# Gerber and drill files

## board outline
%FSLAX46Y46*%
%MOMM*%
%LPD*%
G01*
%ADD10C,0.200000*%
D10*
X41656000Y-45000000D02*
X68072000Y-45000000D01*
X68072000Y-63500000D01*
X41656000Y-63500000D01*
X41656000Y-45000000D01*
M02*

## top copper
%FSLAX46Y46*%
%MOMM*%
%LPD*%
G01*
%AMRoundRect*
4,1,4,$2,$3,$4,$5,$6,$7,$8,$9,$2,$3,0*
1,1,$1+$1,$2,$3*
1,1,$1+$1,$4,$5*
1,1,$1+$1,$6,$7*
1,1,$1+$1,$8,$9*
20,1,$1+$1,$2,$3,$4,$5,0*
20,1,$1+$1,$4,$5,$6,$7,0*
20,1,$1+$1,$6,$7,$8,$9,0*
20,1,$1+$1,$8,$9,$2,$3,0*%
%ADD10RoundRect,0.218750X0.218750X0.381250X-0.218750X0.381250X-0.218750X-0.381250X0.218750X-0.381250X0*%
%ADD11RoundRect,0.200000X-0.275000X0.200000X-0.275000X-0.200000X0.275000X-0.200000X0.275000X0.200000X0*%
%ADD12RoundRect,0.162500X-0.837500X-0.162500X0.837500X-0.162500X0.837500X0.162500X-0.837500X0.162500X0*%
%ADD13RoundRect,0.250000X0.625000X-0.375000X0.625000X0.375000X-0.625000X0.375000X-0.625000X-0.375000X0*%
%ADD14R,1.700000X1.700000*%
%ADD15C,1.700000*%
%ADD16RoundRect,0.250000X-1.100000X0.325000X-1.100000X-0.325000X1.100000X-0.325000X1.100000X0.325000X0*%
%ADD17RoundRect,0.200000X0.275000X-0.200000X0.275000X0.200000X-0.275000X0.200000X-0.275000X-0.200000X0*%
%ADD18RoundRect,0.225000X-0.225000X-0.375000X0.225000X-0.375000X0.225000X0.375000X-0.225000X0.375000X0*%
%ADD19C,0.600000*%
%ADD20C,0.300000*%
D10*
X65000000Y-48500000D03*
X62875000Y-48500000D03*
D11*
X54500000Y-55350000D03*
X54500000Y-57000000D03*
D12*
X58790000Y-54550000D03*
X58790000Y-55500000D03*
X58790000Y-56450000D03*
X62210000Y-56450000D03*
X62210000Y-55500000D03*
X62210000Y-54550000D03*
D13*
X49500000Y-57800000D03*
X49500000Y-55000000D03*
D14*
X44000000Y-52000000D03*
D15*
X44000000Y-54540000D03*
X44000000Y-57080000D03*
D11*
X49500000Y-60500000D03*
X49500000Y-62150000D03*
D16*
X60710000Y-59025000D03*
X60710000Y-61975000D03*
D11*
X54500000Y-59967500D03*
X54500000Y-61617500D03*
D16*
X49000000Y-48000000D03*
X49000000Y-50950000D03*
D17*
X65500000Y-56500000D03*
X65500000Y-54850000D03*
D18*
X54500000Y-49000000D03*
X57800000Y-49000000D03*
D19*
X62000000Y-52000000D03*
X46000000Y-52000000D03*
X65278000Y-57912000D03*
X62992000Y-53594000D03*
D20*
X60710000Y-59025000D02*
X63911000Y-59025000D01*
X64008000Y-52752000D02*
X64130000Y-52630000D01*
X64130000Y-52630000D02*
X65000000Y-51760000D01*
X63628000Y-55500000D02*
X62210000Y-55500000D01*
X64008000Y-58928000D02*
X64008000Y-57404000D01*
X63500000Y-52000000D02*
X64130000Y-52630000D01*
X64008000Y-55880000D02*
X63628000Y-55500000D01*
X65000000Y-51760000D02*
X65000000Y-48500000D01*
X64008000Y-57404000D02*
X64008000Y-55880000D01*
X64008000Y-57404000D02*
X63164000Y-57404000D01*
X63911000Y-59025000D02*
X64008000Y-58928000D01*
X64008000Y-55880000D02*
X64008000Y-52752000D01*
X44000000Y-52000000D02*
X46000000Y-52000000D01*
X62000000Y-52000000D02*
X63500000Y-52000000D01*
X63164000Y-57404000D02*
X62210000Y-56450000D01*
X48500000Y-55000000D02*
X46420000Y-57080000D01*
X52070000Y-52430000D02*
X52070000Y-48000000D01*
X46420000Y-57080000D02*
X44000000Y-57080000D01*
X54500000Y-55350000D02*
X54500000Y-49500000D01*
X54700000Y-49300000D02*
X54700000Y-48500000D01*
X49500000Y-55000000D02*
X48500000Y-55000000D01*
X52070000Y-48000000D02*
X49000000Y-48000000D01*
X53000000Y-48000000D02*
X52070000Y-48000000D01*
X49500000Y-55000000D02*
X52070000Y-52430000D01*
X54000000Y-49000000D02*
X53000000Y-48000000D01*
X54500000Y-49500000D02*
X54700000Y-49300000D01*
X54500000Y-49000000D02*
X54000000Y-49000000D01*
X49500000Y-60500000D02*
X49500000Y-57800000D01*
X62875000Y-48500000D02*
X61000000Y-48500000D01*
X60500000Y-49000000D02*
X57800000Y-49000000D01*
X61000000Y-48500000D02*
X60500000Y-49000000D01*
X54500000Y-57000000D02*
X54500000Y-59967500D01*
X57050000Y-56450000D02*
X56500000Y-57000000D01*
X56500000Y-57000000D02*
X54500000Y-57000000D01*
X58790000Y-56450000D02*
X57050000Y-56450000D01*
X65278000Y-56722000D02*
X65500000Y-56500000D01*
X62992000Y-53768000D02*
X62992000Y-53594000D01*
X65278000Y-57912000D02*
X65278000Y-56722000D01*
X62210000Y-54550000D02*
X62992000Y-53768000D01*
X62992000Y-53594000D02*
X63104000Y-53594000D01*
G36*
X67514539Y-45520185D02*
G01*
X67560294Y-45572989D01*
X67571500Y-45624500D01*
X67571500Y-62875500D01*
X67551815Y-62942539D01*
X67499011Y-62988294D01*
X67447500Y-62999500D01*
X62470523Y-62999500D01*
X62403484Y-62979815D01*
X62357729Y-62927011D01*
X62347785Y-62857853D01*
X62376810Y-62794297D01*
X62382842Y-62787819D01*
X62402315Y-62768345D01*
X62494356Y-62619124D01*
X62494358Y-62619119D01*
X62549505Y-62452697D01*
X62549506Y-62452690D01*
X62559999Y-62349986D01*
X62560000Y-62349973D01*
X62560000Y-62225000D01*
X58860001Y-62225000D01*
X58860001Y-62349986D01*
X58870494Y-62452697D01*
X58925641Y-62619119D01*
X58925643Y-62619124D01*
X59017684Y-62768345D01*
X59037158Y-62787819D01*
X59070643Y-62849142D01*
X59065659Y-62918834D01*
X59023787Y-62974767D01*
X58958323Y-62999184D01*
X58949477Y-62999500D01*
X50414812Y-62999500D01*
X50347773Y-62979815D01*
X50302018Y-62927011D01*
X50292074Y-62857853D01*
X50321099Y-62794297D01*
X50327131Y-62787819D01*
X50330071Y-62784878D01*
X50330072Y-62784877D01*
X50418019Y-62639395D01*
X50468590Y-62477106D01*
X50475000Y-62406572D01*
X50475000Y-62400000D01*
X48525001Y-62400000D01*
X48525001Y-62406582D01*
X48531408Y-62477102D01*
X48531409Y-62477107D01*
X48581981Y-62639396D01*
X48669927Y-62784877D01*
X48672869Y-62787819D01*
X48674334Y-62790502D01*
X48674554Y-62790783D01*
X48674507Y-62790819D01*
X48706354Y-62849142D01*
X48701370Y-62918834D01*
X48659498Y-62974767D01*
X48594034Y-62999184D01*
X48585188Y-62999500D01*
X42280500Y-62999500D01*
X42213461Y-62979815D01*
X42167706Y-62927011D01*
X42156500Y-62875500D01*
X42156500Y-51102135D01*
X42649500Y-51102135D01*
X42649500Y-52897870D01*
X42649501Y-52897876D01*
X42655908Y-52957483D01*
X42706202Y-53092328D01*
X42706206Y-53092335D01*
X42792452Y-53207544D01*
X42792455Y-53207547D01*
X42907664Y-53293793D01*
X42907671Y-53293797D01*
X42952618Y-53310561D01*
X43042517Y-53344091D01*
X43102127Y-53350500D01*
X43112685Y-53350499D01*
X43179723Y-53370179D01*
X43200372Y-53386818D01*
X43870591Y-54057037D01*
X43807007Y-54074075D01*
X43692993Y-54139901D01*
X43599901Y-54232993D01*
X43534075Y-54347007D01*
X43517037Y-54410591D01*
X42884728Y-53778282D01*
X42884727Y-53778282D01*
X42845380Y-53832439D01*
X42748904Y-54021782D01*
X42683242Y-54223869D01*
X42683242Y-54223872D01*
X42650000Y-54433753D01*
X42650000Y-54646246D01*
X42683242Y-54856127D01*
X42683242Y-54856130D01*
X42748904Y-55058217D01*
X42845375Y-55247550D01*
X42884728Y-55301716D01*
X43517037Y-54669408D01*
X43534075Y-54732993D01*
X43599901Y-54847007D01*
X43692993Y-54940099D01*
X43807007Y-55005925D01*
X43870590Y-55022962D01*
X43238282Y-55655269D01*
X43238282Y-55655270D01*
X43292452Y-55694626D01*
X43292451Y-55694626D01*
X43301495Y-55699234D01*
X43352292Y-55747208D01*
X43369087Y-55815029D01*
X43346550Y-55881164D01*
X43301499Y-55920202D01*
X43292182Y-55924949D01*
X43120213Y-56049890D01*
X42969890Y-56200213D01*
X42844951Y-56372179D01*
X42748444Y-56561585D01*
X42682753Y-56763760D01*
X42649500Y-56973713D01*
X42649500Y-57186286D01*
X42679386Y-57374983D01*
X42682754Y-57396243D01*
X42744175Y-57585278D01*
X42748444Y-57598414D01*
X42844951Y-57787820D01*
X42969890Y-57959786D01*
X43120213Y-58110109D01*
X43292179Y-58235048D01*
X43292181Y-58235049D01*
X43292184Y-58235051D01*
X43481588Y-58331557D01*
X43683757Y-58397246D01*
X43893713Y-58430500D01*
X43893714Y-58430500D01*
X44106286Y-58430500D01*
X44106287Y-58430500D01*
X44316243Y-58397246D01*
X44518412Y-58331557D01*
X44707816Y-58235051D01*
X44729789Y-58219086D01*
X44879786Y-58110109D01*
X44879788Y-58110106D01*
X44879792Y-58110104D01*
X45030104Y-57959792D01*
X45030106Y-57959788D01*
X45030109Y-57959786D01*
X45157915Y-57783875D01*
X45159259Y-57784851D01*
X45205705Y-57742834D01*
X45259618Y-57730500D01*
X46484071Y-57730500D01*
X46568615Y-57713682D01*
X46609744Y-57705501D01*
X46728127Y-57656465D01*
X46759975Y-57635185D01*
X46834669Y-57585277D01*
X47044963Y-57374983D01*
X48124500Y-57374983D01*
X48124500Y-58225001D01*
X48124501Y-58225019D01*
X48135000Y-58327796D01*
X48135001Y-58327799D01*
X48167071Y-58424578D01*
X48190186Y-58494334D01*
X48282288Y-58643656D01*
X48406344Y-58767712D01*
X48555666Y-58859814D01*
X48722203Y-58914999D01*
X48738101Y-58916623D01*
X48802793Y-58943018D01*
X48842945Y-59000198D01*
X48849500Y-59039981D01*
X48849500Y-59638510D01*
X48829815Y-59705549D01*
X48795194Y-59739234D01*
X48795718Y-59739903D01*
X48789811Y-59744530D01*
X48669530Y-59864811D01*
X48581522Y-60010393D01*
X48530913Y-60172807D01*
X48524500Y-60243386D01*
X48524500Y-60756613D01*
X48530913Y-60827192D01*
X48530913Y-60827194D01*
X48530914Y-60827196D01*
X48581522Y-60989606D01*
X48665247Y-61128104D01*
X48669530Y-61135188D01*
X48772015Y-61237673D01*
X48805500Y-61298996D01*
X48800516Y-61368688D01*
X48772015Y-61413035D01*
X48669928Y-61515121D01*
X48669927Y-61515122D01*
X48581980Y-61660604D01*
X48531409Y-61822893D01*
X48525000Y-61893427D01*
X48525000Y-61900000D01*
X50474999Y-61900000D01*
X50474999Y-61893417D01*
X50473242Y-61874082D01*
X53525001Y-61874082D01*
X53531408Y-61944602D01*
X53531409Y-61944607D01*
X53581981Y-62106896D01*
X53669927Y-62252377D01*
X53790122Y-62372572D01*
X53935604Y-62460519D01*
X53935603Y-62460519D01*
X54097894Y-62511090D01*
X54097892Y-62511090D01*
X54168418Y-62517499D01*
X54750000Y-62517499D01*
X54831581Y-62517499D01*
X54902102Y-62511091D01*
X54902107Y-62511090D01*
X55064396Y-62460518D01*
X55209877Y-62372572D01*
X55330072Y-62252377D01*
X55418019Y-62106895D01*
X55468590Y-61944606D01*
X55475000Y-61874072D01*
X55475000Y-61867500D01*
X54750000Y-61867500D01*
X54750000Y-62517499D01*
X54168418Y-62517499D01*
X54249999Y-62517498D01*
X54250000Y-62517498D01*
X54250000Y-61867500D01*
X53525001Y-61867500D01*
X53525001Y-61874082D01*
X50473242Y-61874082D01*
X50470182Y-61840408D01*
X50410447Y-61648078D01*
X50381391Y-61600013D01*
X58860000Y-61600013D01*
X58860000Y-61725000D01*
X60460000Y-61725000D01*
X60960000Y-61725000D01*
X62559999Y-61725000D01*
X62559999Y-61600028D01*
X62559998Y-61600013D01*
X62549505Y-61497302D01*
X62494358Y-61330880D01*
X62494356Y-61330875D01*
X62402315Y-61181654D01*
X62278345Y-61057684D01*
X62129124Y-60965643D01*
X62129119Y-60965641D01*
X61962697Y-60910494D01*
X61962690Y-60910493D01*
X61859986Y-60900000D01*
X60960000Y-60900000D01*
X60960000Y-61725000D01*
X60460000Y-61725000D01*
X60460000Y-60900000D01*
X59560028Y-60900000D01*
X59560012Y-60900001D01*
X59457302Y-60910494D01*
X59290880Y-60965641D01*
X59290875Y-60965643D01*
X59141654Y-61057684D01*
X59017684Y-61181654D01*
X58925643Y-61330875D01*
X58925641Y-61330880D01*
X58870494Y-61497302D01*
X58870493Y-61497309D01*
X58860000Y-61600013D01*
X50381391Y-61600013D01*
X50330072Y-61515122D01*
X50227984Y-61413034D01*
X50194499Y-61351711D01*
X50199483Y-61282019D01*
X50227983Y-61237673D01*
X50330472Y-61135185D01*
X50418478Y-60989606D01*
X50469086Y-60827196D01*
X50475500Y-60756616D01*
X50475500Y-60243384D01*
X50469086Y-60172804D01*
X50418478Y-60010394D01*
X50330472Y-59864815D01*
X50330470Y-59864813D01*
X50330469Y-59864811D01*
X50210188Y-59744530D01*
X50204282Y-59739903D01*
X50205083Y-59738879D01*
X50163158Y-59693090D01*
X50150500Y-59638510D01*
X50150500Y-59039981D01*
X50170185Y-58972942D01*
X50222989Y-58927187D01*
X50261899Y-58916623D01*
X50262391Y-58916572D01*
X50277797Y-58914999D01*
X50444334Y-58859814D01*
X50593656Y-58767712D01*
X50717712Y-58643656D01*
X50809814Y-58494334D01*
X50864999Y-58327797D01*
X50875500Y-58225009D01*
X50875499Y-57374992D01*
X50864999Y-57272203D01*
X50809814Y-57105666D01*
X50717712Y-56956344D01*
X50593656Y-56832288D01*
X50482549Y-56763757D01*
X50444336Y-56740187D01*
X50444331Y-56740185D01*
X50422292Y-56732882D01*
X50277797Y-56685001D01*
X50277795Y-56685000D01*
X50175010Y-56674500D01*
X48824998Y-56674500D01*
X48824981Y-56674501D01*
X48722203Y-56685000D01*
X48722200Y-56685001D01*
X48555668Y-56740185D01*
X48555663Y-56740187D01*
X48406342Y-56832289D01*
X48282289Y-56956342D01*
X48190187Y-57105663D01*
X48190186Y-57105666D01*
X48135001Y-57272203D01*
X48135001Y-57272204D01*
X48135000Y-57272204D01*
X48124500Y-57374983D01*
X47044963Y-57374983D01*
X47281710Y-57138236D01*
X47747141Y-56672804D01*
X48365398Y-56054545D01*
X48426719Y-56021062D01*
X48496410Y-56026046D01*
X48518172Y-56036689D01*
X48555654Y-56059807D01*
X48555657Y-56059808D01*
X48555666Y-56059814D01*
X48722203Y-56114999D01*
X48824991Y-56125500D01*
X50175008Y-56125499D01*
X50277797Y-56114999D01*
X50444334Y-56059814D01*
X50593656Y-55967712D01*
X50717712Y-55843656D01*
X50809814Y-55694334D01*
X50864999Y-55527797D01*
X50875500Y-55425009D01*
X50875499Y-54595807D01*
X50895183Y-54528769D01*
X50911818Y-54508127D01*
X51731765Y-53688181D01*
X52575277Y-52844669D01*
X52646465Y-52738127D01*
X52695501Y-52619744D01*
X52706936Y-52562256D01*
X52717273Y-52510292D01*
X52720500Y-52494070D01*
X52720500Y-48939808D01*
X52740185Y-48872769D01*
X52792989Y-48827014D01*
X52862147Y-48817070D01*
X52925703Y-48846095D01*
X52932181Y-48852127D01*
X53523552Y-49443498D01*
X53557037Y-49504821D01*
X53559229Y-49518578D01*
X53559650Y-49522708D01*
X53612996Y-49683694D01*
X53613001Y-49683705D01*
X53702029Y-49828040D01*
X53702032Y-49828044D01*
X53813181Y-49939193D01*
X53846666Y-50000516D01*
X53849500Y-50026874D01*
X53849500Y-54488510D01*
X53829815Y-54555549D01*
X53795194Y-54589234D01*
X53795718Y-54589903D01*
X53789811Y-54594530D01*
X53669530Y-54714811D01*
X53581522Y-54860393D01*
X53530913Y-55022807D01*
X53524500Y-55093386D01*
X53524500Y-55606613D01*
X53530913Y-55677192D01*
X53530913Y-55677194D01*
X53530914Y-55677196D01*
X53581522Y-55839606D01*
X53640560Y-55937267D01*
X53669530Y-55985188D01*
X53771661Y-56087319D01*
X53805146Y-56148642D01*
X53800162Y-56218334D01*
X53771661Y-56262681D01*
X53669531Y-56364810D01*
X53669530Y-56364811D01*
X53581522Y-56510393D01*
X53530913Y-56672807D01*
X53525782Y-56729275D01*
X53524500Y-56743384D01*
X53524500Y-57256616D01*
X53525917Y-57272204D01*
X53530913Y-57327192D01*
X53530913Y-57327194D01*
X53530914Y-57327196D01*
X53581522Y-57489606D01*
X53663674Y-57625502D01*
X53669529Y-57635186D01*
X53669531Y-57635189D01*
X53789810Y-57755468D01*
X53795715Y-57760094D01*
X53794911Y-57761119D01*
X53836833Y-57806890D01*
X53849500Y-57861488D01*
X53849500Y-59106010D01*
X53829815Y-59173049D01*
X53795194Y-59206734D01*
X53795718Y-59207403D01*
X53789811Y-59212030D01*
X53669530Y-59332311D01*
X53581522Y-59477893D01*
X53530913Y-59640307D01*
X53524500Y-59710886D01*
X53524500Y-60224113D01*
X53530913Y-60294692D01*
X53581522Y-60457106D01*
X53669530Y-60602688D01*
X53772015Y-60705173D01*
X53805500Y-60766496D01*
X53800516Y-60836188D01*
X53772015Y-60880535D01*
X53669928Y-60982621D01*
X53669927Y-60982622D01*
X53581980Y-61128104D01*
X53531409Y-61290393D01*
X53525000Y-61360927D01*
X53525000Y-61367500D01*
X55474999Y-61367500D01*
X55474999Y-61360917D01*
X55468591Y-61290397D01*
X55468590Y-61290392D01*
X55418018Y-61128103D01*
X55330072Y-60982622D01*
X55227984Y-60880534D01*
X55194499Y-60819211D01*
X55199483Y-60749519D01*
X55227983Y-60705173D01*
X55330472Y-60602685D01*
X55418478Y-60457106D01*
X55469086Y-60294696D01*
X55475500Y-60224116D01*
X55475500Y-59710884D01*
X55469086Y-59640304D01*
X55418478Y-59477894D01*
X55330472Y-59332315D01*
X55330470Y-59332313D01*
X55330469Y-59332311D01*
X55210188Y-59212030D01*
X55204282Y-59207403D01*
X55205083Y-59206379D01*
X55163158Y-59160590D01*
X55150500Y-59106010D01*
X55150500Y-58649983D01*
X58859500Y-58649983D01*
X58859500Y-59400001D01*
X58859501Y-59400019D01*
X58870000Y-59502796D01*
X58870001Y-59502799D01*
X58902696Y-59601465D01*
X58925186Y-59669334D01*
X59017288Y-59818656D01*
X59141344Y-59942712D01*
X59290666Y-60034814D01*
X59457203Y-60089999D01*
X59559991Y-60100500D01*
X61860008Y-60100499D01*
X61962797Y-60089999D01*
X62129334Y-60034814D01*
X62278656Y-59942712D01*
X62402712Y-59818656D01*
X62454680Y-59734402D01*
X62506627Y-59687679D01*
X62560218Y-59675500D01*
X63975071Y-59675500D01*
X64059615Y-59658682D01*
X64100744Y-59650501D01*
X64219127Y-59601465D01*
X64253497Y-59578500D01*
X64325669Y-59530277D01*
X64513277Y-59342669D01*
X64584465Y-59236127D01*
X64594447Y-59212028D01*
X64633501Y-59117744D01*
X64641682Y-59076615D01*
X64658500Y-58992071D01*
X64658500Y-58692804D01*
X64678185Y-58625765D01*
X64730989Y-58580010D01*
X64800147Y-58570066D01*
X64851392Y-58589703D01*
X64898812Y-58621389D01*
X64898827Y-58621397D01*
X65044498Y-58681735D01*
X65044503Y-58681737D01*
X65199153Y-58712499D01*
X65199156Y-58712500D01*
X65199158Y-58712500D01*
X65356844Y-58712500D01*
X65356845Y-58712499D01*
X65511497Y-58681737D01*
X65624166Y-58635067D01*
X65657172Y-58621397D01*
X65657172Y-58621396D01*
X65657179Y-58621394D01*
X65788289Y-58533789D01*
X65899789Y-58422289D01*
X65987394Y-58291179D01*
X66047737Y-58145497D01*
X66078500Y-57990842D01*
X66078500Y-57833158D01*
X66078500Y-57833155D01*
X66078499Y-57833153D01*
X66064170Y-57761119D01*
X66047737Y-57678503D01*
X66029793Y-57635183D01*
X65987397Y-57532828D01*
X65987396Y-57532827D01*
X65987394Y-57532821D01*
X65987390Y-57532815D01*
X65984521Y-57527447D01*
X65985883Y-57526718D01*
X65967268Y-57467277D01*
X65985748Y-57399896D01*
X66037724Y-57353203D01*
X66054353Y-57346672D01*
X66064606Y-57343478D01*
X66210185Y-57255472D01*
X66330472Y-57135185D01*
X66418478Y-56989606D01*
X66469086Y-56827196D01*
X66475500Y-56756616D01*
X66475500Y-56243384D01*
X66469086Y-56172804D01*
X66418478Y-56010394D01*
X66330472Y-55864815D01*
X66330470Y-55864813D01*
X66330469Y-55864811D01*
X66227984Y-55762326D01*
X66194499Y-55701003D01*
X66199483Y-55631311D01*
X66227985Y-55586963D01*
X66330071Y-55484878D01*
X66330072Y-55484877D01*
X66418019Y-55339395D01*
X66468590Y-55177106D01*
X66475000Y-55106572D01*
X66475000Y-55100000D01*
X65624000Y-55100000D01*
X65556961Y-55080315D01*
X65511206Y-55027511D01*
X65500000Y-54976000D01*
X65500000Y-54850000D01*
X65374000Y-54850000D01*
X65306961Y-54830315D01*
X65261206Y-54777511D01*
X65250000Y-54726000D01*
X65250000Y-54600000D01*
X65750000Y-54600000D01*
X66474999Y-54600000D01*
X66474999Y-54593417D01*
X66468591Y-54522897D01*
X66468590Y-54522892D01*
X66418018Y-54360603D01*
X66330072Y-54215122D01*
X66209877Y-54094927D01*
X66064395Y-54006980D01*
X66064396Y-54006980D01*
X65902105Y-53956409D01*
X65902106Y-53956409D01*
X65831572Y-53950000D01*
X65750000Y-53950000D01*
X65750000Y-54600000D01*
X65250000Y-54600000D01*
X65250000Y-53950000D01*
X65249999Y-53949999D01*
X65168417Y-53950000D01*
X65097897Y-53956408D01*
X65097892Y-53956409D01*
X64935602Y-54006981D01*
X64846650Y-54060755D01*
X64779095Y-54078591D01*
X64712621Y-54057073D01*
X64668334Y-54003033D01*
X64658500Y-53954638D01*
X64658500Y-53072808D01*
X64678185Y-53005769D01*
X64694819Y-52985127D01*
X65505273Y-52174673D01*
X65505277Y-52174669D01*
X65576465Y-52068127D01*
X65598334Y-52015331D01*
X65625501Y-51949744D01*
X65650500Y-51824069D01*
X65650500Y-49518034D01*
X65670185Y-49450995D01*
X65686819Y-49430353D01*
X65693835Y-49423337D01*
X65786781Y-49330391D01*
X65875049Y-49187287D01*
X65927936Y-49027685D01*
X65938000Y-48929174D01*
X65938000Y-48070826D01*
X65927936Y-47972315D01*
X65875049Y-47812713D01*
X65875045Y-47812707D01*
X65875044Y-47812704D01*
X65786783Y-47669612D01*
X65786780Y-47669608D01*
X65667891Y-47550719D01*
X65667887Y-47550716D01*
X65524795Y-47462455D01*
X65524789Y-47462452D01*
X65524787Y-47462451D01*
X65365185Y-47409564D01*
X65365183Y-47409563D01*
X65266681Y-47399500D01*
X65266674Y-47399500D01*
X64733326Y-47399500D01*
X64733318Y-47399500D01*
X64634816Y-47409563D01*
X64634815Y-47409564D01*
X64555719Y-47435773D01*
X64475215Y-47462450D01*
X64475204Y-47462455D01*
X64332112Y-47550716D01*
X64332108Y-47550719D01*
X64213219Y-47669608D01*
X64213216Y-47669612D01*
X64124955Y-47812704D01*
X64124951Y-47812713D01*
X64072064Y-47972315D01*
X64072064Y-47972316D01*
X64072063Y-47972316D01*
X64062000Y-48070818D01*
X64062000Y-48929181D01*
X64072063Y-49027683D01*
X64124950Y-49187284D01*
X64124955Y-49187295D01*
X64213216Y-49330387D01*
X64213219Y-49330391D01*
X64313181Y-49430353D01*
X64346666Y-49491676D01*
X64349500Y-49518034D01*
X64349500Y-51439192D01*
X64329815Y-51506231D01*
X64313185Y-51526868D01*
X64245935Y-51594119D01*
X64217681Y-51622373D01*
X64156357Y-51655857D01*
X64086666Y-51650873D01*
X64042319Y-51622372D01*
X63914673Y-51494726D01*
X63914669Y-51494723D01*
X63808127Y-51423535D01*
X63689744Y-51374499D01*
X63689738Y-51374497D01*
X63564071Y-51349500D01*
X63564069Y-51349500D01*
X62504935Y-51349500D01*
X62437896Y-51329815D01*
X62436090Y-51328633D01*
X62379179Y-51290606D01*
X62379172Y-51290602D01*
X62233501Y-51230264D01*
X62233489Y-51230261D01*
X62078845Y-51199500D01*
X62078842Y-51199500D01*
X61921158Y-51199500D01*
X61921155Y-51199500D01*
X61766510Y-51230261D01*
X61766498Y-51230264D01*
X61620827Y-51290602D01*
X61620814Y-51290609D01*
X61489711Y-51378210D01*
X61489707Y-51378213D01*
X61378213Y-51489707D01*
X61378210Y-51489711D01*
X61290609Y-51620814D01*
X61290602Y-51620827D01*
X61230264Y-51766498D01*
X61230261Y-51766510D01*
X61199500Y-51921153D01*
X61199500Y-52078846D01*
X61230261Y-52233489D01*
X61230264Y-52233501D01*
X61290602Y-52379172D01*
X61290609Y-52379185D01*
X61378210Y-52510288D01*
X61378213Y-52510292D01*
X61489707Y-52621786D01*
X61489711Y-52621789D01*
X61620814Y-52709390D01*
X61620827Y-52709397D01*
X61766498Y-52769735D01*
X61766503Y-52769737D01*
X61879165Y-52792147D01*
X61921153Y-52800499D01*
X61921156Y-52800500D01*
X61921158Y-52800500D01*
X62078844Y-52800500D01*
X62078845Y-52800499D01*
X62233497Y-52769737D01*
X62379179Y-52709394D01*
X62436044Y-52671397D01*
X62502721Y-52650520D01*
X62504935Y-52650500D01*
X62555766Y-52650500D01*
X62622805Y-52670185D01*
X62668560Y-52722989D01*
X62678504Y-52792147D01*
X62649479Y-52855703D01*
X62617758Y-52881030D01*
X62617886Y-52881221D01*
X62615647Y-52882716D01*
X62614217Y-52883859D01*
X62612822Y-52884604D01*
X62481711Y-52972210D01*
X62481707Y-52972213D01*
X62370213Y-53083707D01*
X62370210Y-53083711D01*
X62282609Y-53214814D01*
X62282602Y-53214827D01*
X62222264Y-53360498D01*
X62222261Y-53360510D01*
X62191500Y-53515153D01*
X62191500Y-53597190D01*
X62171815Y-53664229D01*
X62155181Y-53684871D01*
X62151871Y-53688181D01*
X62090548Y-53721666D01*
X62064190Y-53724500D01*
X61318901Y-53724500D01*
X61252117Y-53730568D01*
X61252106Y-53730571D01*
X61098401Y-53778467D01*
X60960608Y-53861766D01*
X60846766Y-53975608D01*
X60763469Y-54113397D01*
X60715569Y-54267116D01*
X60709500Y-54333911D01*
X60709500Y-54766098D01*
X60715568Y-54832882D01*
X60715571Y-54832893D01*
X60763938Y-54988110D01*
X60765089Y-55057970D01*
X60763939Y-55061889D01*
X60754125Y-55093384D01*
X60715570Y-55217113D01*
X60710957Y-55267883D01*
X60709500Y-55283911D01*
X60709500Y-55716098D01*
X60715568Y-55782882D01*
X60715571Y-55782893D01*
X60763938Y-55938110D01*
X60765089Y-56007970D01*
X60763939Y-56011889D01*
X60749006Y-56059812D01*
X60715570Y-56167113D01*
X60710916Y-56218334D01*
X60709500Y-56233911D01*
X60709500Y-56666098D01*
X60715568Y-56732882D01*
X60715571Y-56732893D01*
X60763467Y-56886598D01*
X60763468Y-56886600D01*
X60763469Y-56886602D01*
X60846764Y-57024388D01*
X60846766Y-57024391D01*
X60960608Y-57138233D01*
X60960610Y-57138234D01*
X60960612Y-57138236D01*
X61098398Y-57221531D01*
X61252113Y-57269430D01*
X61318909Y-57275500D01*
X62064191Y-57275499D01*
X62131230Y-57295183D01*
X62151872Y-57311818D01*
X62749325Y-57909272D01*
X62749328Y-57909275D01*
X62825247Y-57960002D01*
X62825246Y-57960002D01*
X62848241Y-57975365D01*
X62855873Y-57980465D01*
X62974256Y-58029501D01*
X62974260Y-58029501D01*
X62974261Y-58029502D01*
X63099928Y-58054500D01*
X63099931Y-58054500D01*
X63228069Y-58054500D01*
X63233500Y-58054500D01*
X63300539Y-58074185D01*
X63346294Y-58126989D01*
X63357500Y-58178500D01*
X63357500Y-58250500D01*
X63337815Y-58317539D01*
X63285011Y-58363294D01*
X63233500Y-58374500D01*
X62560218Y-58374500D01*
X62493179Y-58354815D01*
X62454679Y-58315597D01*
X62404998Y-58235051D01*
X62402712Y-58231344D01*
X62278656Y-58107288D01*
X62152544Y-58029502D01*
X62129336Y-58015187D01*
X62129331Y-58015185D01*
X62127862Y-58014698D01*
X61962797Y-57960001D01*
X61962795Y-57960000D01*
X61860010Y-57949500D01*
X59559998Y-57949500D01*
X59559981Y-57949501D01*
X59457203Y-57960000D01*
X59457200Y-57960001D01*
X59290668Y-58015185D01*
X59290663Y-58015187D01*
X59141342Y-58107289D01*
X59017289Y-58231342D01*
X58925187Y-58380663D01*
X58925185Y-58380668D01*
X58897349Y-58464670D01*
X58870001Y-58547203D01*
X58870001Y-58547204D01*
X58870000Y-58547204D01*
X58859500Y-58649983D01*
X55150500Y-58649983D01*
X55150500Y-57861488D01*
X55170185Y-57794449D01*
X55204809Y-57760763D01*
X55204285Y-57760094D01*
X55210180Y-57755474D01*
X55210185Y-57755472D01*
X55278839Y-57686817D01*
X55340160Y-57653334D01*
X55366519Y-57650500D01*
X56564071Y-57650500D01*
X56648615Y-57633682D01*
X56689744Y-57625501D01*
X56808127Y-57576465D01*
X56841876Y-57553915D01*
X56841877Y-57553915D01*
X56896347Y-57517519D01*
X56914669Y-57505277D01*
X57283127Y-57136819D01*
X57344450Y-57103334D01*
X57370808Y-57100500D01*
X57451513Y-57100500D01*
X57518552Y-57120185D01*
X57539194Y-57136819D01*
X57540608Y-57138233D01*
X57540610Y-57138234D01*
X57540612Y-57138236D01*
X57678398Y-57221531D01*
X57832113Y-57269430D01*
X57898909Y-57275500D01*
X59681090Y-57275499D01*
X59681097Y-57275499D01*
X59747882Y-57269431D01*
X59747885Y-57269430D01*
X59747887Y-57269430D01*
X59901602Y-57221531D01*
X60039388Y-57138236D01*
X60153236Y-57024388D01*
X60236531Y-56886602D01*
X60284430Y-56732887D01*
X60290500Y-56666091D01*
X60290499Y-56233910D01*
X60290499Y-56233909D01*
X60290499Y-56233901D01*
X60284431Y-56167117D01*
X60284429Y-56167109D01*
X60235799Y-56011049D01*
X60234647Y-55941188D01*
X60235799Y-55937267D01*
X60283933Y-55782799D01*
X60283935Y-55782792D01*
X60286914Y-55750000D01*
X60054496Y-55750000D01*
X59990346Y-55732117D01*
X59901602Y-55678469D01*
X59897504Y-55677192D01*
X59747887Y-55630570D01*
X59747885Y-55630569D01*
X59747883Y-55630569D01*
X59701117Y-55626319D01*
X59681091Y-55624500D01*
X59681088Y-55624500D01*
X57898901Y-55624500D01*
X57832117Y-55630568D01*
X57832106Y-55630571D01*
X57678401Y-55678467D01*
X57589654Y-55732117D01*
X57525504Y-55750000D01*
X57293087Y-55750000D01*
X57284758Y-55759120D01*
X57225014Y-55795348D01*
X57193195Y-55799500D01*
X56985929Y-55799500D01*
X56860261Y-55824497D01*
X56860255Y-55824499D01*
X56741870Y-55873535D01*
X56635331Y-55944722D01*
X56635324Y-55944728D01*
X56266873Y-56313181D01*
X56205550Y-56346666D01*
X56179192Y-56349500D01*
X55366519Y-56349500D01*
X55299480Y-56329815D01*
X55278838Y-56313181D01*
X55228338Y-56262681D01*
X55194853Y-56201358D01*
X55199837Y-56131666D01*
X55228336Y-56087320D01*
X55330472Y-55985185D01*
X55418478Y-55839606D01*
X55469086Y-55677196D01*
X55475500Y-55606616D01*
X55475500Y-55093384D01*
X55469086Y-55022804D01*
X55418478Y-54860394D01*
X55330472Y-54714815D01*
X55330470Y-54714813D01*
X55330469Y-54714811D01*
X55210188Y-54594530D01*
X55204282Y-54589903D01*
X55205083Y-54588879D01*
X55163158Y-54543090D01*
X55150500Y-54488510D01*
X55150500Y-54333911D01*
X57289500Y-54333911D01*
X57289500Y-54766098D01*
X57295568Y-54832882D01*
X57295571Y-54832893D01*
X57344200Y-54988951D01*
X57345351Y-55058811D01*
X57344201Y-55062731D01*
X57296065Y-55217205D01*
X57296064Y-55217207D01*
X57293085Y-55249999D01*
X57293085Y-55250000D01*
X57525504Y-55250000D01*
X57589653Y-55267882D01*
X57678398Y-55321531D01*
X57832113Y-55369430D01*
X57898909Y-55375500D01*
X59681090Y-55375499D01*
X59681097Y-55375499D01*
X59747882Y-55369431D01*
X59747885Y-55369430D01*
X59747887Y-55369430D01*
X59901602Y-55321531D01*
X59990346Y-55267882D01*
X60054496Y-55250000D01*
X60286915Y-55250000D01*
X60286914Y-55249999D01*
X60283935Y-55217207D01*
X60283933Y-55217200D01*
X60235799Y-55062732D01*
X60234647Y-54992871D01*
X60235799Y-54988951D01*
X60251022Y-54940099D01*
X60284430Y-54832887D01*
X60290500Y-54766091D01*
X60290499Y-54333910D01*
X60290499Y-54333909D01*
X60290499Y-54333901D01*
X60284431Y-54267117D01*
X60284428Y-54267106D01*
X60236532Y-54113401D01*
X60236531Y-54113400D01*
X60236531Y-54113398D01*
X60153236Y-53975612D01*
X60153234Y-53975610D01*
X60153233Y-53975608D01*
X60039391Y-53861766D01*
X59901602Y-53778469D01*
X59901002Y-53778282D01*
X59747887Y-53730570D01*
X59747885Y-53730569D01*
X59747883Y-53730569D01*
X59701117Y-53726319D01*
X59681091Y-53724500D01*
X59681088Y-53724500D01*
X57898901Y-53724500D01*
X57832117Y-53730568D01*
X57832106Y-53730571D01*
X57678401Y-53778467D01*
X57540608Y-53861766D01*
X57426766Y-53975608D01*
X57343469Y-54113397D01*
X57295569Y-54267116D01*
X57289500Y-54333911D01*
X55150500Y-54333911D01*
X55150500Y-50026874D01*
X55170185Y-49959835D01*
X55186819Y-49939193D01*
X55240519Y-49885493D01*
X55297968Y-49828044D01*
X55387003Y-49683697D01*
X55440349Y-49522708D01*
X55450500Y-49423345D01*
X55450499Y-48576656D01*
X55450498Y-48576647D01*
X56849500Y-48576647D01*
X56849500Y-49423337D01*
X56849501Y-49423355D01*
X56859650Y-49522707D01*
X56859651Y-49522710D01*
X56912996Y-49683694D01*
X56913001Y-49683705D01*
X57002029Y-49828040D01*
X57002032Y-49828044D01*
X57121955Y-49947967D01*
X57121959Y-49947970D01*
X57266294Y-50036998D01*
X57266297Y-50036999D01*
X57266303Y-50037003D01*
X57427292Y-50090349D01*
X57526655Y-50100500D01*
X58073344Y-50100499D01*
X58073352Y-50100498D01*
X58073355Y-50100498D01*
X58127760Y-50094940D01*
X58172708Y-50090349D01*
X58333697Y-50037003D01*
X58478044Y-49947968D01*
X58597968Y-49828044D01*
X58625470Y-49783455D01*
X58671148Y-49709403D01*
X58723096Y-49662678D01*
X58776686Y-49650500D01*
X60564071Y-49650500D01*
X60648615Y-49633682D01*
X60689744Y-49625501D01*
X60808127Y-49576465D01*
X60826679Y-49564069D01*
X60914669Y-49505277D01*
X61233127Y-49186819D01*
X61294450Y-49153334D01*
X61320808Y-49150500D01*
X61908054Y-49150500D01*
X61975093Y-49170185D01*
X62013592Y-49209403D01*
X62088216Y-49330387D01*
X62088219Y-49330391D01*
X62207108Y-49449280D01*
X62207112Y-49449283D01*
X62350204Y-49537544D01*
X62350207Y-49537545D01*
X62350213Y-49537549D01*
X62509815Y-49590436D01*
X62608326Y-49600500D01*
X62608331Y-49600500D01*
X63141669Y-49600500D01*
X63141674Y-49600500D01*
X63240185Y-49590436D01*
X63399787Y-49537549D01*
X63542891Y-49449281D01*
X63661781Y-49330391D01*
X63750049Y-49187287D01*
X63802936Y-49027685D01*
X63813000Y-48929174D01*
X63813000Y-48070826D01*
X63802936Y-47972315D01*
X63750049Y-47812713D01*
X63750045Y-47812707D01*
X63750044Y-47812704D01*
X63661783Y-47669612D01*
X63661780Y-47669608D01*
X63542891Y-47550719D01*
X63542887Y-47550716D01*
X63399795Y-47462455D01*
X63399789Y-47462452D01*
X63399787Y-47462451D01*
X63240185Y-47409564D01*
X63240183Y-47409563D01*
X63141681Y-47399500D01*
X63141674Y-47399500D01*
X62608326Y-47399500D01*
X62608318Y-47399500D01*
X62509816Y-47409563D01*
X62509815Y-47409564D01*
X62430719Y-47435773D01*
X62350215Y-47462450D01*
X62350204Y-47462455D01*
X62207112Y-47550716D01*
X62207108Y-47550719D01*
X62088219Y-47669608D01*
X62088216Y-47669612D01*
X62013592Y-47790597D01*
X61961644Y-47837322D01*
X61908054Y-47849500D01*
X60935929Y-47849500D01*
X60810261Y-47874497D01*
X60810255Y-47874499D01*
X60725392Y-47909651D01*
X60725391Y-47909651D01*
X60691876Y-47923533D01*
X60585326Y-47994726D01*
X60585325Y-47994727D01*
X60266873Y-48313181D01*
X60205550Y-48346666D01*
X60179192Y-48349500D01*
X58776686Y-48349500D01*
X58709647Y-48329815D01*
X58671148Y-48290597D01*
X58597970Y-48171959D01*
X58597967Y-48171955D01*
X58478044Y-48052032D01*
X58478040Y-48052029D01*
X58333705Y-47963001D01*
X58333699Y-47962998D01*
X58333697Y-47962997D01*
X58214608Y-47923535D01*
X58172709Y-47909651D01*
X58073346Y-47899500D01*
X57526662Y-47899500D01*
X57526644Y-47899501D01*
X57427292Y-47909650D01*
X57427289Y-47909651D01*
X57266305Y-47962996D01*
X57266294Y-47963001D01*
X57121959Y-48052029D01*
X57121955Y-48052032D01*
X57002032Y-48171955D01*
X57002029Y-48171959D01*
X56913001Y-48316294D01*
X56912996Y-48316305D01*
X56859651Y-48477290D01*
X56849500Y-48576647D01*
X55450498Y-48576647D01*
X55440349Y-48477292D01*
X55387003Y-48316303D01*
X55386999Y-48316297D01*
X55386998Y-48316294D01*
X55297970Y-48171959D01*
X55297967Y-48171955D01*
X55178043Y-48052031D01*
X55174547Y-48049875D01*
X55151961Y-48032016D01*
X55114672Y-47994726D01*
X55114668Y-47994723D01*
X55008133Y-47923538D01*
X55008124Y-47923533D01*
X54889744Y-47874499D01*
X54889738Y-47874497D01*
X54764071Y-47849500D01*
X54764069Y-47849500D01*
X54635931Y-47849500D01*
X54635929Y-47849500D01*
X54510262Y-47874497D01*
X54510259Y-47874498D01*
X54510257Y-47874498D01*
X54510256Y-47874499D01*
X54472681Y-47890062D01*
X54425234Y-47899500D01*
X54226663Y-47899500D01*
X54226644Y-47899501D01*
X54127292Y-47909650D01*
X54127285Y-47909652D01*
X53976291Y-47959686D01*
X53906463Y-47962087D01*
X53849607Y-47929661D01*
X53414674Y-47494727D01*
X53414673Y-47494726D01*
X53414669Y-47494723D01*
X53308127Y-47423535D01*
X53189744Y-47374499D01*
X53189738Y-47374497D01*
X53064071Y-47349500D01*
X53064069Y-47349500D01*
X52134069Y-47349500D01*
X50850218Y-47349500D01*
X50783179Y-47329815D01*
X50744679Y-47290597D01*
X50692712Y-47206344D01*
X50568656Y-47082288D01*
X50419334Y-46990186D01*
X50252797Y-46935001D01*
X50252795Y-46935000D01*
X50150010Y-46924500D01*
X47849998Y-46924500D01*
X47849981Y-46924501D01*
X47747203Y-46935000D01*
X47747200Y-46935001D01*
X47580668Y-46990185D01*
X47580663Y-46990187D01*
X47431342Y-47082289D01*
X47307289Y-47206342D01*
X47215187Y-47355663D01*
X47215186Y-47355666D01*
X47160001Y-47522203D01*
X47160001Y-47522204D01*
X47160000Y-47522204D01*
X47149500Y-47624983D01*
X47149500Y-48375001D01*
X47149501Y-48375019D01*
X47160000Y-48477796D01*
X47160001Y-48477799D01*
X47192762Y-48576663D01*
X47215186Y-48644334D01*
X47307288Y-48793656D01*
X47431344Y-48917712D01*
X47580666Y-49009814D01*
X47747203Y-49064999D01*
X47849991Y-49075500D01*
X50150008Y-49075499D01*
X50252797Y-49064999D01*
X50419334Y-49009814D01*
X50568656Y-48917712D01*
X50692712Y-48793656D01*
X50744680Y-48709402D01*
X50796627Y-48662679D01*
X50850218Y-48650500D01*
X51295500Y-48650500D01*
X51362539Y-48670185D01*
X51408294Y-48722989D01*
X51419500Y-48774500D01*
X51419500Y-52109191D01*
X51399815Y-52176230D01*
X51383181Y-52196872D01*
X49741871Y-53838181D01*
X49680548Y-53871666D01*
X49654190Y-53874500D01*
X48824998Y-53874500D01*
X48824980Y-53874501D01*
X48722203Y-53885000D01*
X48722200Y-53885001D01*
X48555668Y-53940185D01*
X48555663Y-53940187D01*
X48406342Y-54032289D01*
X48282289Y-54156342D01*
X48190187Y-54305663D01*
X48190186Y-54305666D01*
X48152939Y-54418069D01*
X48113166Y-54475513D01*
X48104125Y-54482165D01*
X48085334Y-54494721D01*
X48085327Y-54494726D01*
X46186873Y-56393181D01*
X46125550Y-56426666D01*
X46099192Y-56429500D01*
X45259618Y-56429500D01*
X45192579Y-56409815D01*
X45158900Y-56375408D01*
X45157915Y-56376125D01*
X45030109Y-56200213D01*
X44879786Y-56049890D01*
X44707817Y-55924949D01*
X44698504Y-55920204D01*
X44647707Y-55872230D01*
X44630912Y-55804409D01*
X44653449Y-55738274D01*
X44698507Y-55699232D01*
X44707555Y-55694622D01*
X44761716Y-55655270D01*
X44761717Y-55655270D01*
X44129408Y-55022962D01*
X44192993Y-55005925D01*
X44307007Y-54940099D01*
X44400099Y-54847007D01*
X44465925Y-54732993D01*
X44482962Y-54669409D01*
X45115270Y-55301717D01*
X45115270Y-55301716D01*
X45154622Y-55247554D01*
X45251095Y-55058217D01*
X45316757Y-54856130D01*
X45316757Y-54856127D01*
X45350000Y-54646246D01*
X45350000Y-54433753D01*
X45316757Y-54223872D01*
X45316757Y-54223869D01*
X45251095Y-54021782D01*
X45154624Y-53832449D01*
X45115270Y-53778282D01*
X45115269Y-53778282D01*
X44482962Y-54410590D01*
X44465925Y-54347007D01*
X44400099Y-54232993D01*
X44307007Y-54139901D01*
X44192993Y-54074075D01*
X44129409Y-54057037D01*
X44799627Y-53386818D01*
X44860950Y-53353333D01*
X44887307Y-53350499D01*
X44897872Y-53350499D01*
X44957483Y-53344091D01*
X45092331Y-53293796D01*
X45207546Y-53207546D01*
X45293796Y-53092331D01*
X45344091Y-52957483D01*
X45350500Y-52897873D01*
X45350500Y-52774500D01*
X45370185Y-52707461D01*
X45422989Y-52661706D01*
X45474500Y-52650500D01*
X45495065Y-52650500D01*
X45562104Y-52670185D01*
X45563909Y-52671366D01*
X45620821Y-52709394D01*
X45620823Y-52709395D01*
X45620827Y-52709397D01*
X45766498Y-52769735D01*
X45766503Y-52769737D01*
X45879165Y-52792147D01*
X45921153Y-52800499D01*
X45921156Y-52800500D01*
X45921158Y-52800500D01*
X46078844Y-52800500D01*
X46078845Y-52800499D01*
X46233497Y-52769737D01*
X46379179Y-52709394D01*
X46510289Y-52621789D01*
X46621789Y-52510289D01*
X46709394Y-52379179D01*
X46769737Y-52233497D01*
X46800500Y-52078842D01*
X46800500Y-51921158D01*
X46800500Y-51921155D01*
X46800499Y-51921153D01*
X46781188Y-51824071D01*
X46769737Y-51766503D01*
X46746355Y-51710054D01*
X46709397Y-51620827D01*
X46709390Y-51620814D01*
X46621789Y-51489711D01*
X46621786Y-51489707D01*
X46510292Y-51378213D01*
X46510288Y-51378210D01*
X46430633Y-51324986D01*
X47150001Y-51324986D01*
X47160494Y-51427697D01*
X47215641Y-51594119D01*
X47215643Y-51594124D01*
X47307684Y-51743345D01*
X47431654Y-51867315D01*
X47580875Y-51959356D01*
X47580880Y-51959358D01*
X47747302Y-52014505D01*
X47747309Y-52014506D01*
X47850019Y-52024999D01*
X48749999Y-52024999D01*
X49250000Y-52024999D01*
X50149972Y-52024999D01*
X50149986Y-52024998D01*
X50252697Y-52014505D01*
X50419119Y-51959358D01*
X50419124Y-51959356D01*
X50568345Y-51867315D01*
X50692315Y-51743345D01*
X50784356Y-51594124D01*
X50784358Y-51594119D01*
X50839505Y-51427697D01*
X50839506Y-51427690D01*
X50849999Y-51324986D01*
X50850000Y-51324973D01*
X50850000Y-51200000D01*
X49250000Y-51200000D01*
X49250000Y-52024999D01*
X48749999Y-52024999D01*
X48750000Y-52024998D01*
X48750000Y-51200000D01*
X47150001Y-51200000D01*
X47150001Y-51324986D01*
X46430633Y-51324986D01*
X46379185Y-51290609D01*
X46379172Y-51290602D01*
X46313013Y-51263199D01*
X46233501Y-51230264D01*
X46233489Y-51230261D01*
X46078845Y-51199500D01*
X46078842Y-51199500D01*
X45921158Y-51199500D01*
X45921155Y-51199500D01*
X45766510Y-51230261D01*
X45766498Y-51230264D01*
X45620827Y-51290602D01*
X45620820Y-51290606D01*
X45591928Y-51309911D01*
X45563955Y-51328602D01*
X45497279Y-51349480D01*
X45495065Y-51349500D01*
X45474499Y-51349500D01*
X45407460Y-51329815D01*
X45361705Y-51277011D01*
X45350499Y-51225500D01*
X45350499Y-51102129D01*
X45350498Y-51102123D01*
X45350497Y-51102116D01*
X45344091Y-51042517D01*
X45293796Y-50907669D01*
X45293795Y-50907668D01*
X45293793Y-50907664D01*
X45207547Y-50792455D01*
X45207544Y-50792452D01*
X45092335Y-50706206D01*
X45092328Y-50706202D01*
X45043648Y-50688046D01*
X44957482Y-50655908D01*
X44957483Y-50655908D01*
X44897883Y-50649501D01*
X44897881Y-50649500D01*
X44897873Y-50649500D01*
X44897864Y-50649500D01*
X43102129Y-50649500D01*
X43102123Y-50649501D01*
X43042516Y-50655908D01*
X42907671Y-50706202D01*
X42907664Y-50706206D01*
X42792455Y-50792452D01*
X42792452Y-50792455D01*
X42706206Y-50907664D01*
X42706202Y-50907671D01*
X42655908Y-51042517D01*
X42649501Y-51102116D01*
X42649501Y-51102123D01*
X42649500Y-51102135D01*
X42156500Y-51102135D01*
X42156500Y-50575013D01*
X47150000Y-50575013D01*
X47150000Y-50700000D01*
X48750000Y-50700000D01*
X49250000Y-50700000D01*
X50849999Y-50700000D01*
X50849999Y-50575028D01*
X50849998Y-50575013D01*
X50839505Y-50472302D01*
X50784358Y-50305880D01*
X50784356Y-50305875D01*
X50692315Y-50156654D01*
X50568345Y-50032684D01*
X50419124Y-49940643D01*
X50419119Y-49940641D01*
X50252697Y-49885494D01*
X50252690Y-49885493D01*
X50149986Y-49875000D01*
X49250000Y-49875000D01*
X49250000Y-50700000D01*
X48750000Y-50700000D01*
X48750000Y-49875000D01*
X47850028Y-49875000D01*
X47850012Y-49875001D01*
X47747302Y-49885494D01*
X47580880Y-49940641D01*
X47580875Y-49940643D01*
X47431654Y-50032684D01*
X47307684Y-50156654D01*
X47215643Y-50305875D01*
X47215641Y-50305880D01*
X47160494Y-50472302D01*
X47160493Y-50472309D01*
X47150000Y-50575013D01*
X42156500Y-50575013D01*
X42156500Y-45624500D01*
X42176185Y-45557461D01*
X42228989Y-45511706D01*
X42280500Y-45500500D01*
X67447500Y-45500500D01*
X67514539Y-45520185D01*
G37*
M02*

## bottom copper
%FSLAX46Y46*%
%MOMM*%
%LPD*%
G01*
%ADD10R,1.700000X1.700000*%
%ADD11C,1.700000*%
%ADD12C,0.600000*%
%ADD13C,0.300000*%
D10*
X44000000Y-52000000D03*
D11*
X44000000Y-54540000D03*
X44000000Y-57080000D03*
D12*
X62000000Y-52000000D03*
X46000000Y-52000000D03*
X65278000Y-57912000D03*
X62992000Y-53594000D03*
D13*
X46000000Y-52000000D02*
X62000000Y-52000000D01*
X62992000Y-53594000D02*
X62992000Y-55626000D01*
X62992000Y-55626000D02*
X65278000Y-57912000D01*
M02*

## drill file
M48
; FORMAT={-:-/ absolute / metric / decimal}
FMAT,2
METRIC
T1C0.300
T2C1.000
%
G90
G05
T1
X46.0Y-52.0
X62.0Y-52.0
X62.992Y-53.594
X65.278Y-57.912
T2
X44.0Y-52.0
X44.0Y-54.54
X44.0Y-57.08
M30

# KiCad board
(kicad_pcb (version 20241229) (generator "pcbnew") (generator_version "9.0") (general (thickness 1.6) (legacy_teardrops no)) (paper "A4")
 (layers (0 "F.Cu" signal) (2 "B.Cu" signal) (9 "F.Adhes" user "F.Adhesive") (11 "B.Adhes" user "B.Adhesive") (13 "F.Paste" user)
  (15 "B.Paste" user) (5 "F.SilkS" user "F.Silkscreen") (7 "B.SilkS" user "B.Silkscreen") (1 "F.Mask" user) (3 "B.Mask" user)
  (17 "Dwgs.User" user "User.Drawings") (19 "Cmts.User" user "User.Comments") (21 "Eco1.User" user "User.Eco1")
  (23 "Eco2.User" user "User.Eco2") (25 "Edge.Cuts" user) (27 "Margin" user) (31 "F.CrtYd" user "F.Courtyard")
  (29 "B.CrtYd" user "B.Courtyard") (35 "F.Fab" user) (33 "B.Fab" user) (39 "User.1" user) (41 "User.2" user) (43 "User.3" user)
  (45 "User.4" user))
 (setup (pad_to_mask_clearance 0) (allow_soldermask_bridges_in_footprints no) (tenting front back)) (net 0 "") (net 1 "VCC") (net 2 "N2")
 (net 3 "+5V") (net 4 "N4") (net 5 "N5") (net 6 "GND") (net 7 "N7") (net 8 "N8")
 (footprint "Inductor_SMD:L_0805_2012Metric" (layer "F.Cu") (at 63.9375 48.5 180)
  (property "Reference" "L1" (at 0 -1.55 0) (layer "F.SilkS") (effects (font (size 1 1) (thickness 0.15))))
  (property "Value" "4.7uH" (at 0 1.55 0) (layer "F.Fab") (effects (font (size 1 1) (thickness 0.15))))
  (pad "1" smd roundrect (at -1.0625 0 180) (size 0.875 1.2) (layers "F.Cu" "F.Mask" "F.Paste") (roundrect_rratio 0.25) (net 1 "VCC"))
  (pad "2" smd roundrect (at 1.0625 0 180) (size 0.875 1.2) (layers "F.Cu" "F.Mask" "F.Paste") (roundrect_rratio 0.25) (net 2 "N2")))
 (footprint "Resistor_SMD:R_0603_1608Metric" (layer "F.Cu") (at 54.5 56.175 -90)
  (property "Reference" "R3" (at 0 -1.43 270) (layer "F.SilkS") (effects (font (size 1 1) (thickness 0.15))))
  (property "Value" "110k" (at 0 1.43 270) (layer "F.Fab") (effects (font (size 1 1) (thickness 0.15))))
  (pad "1" smd roundrect (at -0.825 0 270) (size 0.8 0.95) (layers "F.Cu" "F.Mask" "F.Paste") (roundrect_rratio 0.25) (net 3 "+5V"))
  (pad "2" smd roundrect (at 0.825 0 270) (size 0.8 0.95) (layers "F.Cu" "F.Mask" "F.Paste") (roundrect_rratio 0.25) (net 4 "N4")))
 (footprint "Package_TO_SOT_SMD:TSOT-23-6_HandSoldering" (layer "F.Cu") (at 60.5 55.5)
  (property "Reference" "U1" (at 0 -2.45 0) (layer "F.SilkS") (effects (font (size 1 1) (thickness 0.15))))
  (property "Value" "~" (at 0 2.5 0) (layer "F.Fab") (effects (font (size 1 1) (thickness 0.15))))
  (pad "1" smd roundrect (at -1.71 -0.95) (size 2 0.65) (layers "F.Cu" "F.Mask" "F.Paste") (roundrect_rratio 0.25) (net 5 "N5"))
  (pad "2" smd roundrect (at -1.71 0) (size 2 0.65) (layers "F.Cu" "F.Mask" "F.Paste") (roundrect_rratio 0.25) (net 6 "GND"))
  (pad "3" smd roundrect (at -1.71 0.95) (size 2 0.65) (layers "F.Cu" "F.Mask" "F.Paste") (roundrect_rratio 0.25) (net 4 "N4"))
  (pad "4" smd roundrect (at 1.71 0.95) (size 2 0.65) (layers "F.Cu" "F.Mask" "F.Paste") (roundrect_rratio 0.25) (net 1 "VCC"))
  (pad "5" smd roundrect (at 1.71 0) (size 2 0.65) (layers "F.Cu" "F.Mask" "F.Paste") (roundrect_rratio 0.25) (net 1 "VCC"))
  (pad "6" smd roundrect (at 1.71 -0.95) (size 2 0.65) (layers "F.Cu" "F.Mask" "F.Paste") (roundrect_rratio 0.25) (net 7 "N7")))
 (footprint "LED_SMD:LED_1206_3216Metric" (layer "F.Cu") (at 49.5 56.4 90)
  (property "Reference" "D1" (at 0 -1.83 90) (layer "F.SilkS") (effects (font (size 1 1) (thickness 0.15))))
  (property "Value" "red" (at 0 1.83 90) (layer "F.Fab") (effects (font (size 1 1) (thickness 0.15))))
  (pad "1" smd roundrect (at -1.4 0 90) (size 1.25 1.75) (layers "F.Cu" "F.Mask" "F.Paste") (roundrect_rratio 0.2) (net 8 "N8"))
  (pad "2" smd roundrect (at 1.4 0 90) (size 1.25 1.75) (layers "F.Cu" "F.Mask" "F.Paste") (roundrect_rratio 0.2) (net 3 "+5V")))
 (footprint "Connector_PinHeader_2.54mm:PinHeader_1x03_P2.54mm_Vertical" (layer "F.Cu") (at 44 52)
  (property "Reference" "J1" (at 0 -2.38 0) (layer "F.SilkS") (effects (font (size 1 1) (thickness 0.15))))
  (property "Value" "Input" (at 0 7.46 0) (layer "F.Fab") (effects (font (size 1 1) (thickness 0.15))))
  (pad "1" thru_hole rect (at 0 0) (size 1.7 1.7) (drill 1) (layers "*.Cu" "*.Mask") (remove_unused_layers no) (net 1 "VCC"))
  (pad "2" thru_hole circle (at 0 2.54) (size 1.7 1.7) (drill 1) (layers "*.Cu" "*.Mask") (remove_unused_layers no) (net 6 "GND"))
  (pad "3" thru_hole circle (at 0 5.08) (size 1.7 1.7) (drill 1) (layers "*.Cu" "*.Mask") (remove_unused_layers no) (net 3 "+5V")))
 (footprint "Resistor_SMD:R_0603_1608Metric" (layer "F.Cu") (at 49.5 61.325 -90)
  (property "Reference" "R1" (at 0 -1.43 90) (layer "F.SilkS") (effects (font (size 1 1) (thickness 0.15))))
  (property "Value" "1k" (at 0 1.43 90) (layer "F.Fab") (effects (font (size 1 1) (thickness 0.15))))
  (pad "1" smd roundrect (at -0.825 0 270) (size 0.8 0.95) (layers "F.Cu" "F.Mask" "F.Paste") (roundrect_rratio 0.25) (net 8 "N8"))
  (pad "2" smd roundrect (at 0.825 0 270) (size 0.8 0.95) (layers "F.Cu" "F.Mask" "F.Paste") (roundrect_rratio 0.25) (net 6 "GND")))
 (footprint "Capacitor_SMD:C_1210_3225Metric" (layer "F.Cu") (at 60.71 60.5 -90)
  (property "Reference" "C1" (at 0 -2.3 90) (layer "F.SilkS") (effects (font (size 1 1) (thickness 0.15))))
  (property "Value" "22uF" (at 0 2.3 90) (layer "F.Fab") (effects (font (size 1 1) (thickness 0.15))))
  (pad "1" smd roundrect (at -1.475 0 270) (size 1.15 2.7) (layers "F.Cu" "F.Mask" "F.Paste") (roundrect_rratio 0.217391) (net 1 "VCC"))
  (pad "2" smd roundrect (at 1.475 0 270) (size 1.15 2.7) (layers "F.Cu" "F.Mask" "F.Paste") (roundrect_rratio 0.217391) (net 6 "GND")))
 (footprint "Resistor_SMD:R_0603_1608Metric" (layer "F.Cu") (at 54.5 60.7925 -90)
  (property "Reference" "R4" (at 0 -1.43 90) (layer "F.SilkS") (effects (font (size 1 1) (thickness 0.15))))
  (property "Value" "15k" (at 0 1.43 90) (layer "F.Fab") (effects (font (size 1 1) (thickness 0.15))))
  (pad "1" smd roundrect (at -0.825 0 270) (size 0.8 0.95) (layers "F.Cu" "F.Mask" "F.Paste") (roundrect_rratio 0.25) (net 4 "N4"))
  (pad "2" smd roundrect (at 0.825 0 270) (size 0.8 0.95) (layers "F.Cu" "F.Mask" "F.Paste") (roundrect_rratio 0.25) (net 6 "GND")))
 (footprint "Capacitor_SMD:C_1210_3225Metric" (layer "F.Cu") (at 49 49.475 -90)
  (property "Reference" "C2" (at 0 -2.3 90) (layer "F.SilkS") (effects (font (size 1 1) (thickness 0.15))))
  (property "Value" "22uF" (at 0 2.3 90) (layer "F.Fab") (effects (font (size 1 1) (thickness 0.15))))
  (pad "1" smd roundrect (at -1.475 0 270) (size 1.15 2.7) (layers "F.Cu" "F.Mask" "F.Paste") (roundrect_rratio 0.217391) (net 3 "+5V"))
  (pad "2" smd roundrect (at 1.475 0 270) (size 1.15 2.7) (layers "F.Cu" "F.Mask" "F.Paste") (roundrect_rratio 0.217391) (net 6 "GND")))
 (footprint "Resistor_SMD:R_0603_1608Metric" (layer "F.Cu") (at 65.5 55.675 90)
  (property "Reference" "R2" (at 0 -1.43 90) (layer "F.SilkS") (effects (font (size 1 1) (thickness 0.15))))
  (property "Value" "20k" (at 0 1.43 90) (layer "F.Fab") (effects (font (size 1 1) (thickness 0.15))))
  (pad "1" smd roundrect (at -0.825 0 90) (size 0.8 0.95) (layers "F.Cu" "F.Mask" "F.Paste") (roundrect_rratio 0.25) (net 7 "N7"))
  (pad "2" smd roundrect (at 0.825 0 90) (size 0.8 0.95) (layers "F.Cu" "F.Mask" "F.Paste") (roundrect_rratio 0.25) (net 6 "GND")))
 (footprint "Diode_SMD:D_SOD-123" (layer "F.Cu") (at 56.15 49)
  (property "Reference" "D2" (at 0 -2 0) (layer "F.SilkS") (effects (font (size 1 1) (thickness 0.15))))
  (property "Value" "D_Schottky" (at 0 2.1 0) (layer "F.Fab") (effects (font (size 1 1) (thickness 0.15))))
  (pad "1" smd roundrect (at -1.65 0) (size 0.9 1.2) (layers "F.Cu" "F.Mask" "F.Paste") (roundrect_rratio 0.25) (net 3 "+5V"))
  (pad "2" smd roundrect (at 1.65 0) (size 0.9 1.2) (layers "F.Cu" "F.Mask" "F.Paste") (roundrect_rratio 0.25) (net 2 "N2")))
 (gr_rect (start 41.656 45) (end 68.072 63.5) (stroke (width 0.2) (type solid)) (fill no) (layer "Edge.Cuts"))
 (segment (start 60.71 59.025) (end 63.911 59.025) (width 0.3) (layer "F.Cu") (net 1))
 (segment (start 64.008 52.752) (end 64.13 52.63) (width 0.3) (layer "F.Cu") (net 1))
 (segment (start 64.13 52.63) (end 65 51.76) (width 0.3) (layer "F.Cu") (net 1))
 (segment (start 63.628 55.5) (end 62.21 55.5) (width 0.3) (layer "F.Cu") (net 1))
 (segment (start 64.008 58.928) (end 64.008 57.404) (width 0.3) (layer "F.Cu") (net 1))
 (segment (start 63.5 52) (end 64.13 52.63) (width 0.3) (layer "F.Cu") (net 1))
 (segment (start 64.008 55.88) (end 63.628 55.5) (width 0.3) (layer "F.Cu") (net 1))
 (segment (start 65 51.76) (end 65 48.5) (width 0.3) (layer "F.Cu") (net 1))
 (segment (start 64.008 57.404) (end 64.008 55.88) (width 0.3) (layer "F.Cu") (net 1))
 (segment (start 64.008 57.404) (end 63.164 57.404) (width 0.3) (layer "F.Cu") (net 1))
 (segment (start 63.911 59.025) (end 64.008 58.928) (width 0.3) (layer "F.Cu") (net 1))
 (segment (start 64.008 55.88) (end 64.008 52.752) (width 0.3) (layer "F.Cu") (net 1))
 (segment (start 44 52) (end 46 52) (width 0.3) (layer "F.Cu") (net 1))
 (segment (start 62 52) (end 63.5 52) (width 0.3) (layer "F.Cu") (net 1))
 (segment (start 63.164 57.404) (end 62.21 56.45) (width 0.3) (layer "F.Cu") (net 1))
 (via (at 62 52) (size 0.6) (drill 0.3) (layers "F.Cu" "B.Cu") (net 1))
 (via (at 46 52) (size 0.6) (drill 0.3) (layers "F.Cu" "B.Cu") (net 1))
 (segment (start 46 52) (end 62 52) (width 0.3) (layer "B.Cu") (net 1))
 (segment (start 48.5 55) (end 46.42 57.08) (width 0.3) (layer "F.Cu") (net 3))
 (segment (start 52.07 52.43) (end 52.07 48) (width 0.3) (layer "F.Cu") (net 3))
 (segment (start 46.42 57.08) (end 44 57.08) (width 0.3) (layer "F.Cu") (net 3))
 (segment (start 54.5 55.35) (end 54.5 49.5) (width 0.3) (layer "F.Cu") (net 3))
 (segment (start 54.7 49.3) (end 54.7 48.5) (width 0.3) (layer "F.Cu") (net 3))
 (segment (start 49.5 55) (end 48.5 55) (width 0.3) (layer "F.Cu") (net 3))
 (segment (start 52.07 48) (end 49 48) (width 0.3) (layer "F.Cu") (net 3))
 (segment (start 53 48) (end 52.07 48) (width 0.3) (layer "F.Cu") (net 3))
 (segment (start 49.5 55) (end 52.07 52.43) (width 0.3) (layer "F.Cu") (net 3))
 (segment (start 54 49) (end 53 48) (width 0.3) (layer "F.Cu") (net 3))
 (segment (start 54.5 49.5) (end 54.7 49.3) (width 0.3) (layer "F.Cu") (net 3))
 (segment (start 54.5 49) (end 54 49) (width 0.3) (layer "F.Cu") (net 3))
 (segment (start 49.5 60.5) (end 49.5 57.8) (width 0.3) (layer "F.Cu") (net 8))
 (segment (start 62.875 48.5) (end 61 48.5) (width 0.3) (layer "F.Cu") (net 2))
 (segment (start 60.5 49) (end 57.8 49) (width 0.3) (layer "F.Cu") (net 2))
 (segment (start 61 48.5) (end 60.5 49) (width 0.3) (layer "F.Cu") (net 2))
 (segment (start 54.5 57) (end 54.5 59.9675) (width 0.3) (layer "F.Cu") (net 4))
 (segment (start 57.05 56.45) (end 56.5 57) (width 0.3) (layer "F.Cu") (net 4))
 (segment (start 56.5 57) (end 54.5 57) (width 0.3) (layer "F.Cu") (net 4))
 (segment (start 58.79 56.45) (end 57.05 56.45) (width 0.3) (layer "F.Cu") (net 4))
 (segment (start 65.278 56.722) (end 65.5 56.5) (width 0.3) (layer "F.Cu") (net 7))
 (segment (start 62.992 53.768) (end 62.992 53.594) (width 0.3) (layer "F.Cu") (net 7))
 (segment (start 65.278 57.912) (end 65.278 56.722) (width 0.3) (layer "F.Cu") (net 7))
 (segment (start 62.21 54.55) (end 62.992 53.768) (width 0.3) (layer "F.Cu") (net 7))
 (segment (start 62.992 53.594) (end 63.104 53.594) (width 0.3) (layer "F.Cu") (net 7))
 (via (at 65.278 57.912) (size 0.6) (drill 0.3) (layers "F.Cu" "B.Cu") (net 7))
 (via (at 62.992 53.594) (size 0.6) (drill 0.3) (layers "F.Cu" "B.Cu") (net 7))
 (segment (start 62.992 53.594) (end 62.992 55.626) (width 0.3) (layer "B.Cu") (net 7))
 (segment (start 62.992 55.626) (end 65.278 57.912) (width 0.3) (layer "B.Cu") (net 7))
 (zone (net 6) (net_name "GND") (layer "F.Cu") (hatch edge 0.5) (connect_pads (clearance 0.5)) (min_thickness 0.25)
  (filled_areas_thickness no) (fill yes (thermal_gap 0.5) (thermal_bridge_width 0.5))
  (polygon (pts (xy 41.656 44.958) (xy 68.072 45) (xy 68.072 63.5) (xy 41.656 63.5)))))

